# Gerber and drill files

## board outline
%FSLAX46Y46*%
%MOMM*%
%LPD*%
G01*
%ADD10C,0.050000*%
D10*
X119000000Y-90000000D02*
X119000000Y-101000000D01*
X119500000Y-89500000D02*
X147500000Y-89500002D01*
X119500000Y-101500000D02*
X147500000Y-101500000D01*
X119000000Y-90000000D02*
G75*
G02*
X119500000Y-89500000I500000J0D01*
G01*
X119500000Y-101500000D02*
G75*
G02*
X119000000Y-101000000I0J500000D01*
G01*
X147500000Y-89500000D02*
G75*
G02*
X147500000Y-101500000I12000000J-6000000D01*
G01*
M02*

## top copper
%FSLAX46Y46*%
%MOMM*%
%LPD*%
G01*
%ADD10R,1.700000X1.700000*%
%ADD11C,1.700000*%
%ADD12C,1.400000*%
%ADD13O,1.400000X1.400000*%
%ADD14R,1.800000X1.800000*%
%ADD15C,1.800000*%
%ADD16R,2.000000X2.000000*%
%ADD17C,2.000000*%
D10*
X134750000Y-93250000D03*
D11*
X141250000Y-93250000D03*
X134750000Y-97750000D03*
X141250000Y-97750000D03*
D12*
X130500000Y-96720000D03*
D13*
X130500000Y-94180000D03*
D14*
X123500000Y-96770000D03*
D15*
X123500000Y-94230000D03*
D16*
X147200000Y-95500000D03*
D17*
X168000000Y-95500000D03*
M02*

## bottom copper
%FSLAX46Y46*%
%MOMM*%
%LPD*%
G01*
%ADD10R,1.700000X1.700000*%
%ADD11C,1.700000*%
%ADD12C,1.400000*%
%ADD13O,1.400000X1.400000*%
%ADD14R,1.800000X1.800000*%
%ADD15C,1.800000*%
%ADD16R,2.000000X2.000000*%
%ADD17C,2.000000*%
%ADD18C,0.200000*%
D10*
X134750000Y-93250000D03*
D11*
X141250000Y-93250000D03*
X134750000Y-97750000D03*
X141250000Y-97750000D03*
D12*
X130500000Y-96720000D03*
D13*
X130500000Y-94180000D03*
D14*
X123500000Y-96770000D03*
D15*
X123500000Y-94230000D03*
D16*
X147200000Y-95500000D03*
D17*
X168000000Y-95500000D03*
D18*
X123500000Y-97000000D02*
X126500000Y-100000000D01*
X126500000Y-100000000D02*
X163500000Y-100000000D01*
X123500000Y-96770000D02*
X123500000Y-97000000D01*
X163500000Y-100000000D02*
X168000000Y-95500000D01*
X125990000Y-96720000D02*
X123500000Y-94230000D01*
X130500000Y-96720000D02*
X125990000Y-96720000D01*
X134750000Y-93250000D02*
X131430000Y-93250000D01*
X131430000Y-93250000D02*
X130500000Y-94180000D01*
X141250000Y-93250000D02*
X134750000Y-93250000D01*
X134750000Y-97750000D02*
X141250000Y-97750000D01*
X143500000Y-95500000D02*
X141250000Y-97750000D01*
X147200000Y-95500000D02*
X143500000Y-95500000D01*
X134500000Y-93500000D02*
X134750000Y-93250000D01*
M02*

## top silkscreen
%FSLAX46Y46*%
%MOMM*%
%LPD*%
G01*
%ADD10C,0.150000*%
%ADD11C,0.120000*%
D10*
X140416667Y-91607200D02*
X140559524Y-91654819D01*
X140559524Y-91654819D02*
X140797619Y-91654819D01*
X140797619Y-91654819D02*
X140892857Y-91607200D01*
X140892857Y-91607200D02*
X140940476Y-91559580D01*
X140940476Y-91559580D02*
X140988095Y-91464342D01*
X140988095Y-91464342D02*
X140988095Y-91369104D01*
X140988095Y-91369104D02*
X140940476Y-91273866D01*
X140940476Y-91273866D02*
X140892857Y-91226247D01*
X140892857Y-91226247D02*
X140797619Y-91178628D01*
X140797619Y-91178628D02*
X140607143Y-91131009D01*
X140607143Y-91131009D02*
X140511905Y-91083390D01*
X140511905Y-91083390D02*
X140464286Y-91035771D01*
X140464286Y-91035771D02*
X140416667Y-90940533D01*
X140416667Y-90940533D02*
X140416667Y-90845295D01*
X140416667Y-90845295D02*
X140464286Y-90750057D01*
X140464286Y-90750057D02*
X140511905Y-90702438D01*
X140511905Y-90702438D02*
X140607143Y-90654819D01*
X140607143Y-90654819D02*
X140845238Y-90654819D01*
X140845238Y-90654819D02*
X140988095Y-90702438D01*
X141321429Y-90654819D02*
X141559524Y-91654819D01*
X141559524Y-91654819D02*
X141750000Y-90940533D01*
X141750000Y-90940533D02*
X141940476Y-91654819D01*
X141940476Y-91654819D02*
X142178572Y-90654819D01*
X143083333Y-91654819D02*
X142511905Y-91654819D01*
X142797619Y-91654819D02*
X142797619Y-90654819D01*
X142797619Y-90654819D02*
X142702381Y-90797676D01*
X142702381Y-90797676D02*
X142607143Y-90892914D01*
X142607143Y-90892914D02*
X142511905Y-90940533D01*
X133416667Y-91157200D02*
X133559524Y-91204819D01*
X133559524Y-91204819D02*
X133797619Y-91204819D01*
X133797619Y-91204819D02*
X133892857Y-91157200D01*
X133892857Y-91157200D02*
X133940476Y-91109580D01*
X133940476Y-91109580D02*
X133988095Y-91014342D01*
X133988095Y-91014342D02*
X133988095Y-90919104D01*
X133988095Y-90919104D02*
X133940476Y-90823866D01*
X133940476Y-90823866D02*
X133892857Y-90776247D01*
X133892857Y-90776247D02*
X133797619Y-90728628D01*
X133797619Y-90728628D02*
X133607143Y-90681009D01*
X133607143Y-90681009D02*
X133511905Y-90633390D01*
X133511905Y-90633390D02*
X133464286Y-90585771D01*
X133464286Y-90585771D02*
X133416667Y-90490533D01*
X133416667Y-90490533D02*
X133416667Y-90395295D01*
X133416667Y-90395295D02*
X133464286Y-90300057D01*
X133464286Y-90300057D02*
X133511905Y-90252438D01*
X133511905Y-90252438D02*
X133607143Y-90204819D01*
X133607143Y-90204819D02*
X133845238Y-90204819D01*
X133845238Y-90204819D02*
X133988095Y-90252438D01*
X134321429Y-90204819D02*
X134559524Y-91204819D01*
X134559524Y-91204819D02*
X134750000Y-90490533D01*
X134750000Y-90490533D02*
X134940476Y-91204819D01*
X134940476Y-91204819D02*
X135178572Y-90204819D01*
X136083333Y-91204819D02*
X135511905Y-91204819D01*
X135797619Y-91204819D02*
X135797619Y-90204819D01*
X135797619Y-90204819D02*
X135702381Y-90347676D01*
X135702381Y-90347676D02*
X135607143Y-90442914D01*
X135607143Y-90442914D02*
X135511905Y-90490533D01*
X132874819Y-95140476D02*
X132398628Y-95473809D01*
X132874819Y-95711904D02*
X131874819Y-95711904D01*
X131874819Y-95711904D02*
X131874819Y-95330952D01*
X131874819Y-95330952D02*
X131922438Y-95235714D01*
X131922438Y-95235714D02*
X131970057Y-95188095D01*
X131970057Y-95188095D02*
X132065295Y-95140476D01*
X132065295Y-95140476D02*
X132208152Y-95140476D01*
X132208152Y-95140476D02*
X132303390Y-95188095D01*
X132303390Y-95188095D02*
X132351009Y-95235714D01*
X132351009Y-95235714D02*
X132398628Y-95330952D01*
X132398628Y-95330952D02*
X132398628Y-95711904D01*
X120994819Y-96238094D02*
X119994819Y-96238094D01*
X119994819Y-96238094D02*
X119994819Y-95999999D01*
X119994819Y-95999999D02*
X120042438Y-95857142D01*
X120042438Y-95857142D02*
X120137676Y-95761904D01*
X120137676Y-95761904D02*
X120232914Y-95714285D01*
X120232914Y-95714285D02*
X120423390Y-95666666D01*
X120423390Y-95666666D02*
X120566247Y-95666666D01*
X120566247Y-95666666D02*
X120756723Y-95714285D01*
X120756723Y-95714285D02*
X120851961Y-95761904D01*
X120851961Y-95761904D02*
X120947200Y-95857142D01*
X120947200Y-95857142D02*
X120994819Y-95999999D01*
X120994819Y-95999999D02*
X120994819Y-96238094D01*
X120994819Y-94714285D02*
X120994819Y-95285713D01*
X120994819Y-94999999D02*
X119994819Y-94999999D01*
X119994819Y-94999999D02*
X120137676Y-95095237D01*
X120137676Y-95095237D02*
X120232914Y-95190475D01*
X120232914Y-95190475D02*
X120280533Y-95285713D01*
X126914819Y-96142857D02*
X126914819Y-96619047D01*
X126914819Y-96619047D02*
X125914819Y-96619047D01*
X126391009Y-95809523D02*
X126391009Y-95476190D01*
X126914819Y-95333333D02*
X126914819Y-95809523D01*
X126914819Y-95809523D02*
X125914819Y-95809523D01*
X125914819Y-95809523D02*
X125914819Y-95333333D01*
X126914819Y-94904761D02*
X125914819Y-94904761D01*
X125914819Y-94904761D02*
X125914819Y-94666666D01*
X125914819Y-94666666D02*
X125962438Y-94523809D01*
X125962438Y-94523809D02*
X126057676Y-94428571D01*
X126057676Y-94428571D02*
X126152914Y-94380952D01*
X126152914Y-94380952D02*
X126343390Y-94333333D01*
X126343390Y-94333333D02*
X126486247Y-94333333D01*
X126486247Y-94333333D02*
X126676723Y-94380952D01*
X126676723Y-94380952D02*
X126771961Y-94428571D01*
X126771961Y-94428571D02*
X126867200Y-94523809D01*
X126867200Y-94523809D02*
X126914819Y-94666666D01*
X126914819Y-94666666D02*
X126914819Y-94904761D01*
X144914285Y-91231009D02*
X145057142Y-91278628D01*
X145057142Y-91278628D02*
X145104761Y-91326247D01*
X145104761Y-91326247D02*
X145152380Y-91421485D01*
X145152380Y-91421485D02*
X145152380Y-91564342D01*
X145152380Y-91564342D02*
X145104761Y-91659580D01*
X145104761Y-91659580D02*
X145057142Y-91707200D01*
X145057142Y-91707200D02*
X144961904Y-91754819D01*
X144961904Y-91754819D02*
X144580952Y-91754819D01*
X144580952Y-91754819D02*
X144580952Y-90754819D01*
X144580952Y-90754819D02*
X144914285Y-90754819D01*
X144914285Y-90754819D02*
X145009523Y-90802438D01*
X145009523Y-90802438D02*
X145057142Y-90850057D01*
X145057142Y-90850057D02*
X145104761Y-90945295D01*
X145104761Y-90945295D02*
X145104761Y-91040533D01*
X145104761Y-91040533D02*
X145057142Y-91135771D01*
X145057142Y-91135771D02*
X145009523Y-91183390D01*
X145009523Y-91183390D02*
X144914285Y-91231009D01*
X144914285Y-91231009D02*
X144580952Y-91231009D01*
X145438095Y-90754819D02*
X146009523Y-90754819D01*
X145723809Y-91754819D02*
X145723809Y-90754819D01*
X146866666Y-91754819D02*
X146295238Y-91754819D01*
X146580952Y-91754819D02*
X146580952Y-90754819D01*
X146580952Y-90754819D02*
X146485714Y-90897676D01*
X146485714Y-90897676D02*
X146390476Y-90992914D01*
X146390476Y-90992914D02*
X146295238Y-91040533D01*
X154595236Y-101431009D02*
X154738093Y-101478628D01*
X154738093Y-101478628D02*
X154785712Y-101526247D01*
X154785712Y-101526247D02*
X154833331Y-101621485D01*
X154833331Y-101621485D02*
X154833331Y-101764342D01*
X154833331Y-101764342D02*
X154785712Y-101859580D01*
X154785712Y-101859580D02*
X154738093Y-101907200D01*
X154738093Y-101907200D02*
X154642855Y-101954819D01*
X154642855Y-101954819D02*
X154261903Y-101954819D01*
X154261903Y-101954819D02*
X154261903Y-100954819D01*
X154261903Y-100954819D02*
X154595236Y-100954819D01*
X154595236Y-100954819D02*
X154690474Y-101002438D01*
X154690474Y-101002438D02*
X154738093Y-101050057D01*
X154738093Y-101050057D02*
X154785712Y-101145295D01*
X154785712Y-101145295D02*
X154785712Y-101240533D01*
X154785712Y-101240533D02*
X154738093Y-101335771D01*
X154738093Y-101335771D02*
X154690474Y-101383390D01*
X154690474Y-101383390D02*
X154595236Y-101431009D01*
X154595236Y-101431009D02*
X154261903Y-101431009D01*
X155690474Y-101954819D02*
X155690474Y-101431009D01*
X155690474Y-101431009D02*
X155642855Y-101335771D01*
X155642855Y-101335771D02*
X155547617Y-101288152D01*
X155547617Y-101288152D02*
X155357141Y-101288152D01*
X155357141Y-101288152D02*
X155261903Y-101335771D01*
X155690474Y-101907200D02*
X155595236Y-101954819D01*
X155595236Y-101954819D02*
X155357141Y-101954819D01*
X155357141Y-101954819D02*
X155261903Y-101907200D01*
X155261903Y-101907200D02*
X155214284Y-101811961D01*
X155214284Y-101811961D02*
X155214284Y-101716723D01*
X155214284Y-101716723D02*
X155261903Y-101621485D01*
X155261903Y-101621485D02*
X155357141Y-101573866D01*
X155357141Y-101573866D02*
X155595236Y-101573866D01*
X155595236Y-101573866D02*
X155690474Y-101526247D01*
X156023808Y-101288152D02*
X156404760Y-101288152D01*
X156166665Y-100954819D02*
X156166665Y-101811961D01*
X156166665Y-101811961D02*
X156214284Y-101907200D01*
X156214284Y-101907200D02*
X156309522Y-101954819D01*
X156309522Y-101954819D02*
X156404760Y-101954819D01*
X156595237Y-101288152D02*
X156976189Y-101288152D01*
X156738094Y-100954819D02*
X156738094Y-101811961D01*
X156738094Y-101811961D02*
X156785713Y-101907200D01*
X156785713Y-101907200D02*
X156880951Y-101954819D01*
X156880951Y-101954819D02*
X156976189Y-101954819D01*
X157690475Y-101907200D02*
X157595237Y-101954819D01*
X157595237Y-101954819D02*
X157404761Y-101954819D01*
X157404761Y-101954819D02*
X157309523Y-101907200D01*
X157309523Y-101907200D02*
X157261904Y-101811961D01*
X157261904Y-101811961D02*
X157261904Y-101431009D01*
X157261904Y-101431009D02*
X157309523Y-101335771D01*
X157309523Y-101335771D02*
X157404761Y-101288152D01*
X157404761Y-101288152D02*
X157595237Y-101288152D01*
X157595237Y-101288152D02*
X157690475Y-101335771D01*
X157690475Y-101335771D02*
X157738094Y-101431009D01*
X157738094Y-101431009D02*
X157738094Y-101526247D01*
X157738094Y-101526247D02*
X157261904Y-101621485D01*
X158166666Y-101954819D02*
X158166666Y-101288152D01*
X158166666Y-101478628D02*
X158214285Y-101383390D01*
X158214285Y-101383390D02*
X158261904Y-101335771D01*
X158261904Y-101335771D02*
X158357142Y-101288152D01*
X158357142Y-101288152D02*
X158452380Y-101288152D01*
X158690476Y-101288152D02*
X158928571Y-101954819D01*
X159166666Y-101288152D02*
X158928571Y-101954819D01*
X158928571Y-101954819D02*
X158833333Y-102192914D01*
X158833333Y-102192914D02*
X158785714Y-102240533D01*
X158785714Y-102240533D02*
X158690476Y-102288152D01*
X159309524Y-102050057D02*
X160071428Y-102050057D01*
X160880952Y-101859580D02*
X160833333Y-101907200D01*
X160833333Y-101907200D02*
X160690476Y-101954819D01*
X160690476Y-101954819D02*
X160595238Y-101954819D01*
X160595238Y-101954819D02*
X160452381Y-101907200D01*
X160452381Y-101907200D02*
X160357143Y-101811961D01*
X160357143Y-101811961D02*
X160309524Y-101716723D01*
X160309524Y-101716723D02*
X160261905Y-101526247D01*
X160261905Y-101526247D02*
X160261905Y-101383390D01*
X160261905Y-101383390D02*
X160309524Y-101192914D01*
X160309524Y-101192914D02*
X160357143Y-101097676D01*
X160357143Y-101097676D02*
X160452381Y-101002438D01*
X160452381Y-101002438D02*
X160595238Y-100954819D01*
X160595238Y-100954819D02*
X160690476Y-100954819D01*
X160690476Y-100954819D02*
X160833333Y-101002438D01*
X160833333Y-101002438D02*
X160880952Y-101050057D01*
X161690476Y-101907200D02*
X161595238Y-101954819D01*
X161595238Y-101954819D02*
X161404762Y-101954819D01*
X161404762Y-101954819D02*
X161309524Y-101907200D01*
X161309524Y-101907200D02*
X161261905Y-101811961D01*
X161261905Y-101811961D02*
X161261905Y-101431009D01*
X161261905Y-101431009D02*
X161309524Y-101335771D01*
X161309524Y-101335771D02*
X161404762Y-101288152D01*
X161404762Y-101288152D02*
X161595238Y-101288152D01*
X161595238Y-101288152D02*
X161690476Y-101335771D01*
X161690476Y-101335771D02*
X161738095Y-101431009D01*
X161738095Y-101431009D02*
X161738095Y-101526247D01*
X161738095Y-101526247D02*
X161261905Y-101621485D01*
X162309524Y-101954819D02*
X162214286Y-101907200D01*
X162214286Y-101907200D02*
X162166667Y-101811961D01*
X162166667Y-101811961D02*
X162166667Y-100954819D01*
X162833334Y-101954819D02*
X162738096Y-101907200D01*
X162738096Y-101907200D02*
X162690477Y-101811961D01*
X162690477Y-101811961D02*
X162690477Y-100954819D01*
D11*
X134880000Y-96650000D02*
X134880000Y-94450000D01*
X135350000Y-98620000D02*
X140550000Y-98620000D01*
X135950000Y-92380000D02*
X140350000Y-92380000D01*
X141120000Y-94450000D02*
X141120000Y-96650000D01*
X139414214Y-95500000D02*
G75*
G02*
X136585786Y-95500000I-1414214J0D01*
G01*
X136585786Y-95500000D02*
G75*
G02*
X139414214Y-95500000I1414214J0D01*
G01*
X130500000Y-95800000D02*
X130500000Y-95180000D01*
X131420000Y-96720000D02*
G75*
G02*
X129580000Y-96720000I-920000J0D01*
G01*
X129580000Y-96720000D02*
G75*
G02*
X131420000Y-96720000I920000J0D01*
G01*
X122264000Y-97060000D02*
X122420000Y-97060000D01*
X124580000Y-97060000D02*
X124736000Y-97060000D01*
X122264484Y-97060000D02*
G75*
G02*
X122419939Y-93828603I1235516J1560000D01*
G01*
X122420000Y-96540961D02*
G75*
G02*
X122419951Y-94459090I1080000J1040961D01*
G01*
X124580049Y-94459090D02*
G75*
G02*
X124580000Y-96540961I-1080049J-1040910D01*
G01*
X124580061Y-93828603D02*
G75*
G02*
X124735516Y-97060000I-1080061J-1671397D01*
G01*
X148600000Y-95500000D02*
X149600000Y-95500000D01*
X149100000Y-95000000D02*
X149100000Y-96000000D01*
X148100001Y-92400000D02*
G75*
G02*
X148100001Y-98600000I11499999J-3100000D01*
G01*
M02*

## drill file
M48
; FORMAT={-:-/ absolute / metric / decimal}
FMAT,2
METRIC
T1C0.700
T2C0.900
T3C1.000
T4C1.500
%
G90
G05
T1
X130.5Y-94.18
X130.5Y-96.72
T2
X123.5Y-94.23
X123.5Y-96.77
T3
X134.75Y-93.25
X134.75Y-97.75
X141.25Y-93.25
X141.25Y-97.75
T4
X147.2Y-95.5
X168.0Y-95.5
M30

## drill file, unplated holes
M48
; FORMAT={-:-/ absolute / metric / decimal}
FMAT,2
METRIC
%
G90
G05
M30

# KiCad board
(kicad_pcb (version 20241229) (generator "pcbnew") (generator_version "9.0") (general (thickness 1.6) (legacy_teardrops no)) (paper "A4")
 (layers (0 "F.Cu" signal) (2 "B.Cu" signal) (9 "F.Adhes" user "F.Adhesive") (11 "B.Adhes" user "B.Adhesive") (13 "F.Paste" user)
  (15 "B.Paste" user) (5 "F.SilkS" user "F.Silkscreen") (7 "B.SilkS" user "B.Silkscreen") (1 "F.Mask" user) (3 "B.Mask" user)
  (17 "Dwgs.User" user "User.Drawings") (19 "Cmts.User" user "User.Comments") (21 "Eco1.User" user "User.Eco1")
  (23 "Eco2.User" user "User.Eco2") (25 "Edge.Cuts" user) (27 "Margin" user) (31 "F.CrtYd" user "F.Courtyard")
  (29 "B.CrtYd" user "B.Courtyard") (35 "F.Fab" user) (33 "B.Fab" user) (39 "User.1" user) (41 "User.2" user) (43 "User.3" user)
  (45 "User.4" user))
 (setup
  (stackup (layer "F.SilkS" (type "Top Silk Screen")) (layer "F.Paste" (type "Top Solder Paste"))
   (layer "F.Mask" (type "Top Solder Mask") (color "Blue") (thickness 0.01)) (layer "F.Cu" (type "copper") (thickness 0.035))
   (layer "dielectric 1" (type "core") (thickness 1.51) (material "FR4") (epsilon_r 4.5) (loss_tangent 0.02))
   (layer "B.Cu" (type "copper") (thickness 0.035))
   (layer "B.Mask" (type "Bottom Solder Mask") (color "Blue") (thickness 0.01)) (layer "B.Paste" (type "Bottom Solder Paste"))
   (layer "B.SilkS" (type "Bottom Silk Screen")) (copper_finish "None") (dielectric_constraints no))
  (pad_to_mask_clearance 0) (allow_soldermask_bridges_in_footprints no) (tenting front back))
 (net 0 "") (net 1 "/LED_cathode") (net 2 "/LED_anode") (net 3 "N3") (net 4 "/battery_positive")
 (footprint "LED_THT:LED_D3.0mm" (layer "F.Cu") (at 123.5 96.77 90)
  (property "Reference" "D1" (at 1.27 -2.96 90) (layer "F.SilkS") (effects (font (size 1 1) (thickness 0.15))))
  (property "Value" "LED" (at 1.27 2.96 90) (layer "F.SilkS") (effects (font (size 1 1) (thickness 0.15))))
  (fp_line (start -0.29 -1.236) (end -0.29 -1.08) (stroke (width 0.12) (type solid)) (layer "F.SilkS"))
  (fp_line (start -0.29 1.08) (end -0.29 1.236) (stroke (width 0.12) (type solid)) (layer "F.SilkS"))
  (fp_arc (start -0.29 -1.235516) (mid 1.365624 -1.987701) (end 2.941397 -1.080061) (stroke (width 0.12) (type solid)) (layer "F.SilkS"))
  (fp_arc (start 0.229039 -1.08) (mid 1.269964 -1.5) (end 2.31091 -1.080049) (stroke (width 0.12) (type solid)) (layer "F.SilkS"))
  (fp_arc (start 2.31091 1.080049) (mid 1.269964 1.5) (end 0.229039 1.08) (stroke (width 0.12) (type solid)) (layer "F.SilkS"))
  (fp_arc (start 2.941397 1.080061) (mid 1.365624 1.987701) (end -0.29 1.235516) (stroke (width 0.12) (type solid)) (layer "F.SilkS"))
  (pad "1" thru_hole rect (at 0 0 90) (size 1.8 1.8) (drill 0.9) (layers "*.Cu" "*.Mask") (remove_unused_layers no) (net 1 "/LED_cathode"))
  (pad "2" thru_hole circle (at 2.54 0 90) (size 1.8 1.8) (drill 0.9) (layers "*.Cu" "*.Mask") (remove_unused_layers no)
   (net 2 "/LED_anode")))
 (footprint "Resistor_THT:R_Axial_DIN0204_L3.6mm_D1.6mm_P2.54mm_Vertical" (layer "F.Cu") (at 130.5 96.72 90)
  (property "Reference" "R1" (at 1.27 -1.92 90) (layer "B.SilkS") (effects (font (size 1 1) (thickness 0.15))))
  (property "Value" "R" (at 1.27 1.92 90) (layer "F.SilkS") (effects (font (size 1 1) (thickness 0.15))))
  (fp_line (start 0.92 0) (end 1.54 0) (stroke (width 0.12) (type solid)) (layer "F.SilkS"))
  (fp_circle (center 0 0) (end 0.92 0) (stroke (width 0.12) (type solid)) (fill no) (layer "F.SilkS"))
  (pad "1" thru_hole circle (at 0 0 90) (size 1.4 1.4) (drill 0.7) (layers "*.Cu" "*.Mask") (remove_unused_layers no) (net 2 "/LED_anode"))
  (pad "2" thru_hole oval (at 2.54 0 90) (size 1.4 1.4) (drill 0.7) (layers "*.Cu" "*.Mask") (remove_unused_layers no) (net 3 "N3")))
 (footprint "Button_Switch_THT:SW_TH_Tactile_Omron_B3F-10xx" (layer "F.Cu") (at 134.75 93.25)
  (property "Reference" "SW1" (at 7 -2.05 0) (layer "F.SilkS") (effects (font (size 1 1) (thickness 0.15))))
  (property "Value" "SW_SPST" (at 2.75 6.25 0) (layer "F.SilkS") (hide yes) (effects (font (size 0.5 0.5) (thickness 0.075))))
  (fp_line (start 0.13 3.4) (end 0.13 1.2) (stroke (width 0.12) (type solid)) (layer "F.SilkS"))
  (fp_line (start 0.6 5.37) (end 5.8 5.37) (stroke (width 0.12) (type solid)) (layer "F.SilkS"))
  (fp_line (start 1.2 -0.87) (end 5.6 -0.87) (stroke (width 0.12) (type solid)) (layer "F.SilkS"))
  (fp_line (start 6.37 1.2) (end 6.37 3.4) (stroke (width 0.12) (type solid)) (layer "F.SilkS"))
  (fp_circle (center 3.25 2.25) (end 4.25 3.25) (stroke (width 0.12) (type solid)) (fill no) (layer "F.SilkS"))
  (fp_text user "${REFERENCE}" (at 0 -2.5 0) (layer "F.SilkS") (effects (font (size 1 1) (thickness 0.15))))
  (pad "1" thru_hole rect (at 0 0) (size 1.7 1.7) (drill 1) (layers "*.Cu" "*.Mask") (remove_unused_layers no) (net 3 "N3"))
  (pad "1" thru_hole circle (at 6.5 0) (size 1.7 1.7) (drill 1) (layers "*.Cu" "*.Mask") (remove_unused_layers no) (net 3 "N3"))
  (pad "2" thru_hole circle (at 0 4.5) (size 1.7 1.7) (drill 1) (layers "*.Cu" "*.Mask") (remove_unused_layers no)
   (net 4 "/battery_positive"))
  (pad "2" thru_hole circle (at 6.5 4.5) (size 1.7 1.7) (drill 1) (layers "*.Cu" "*.Mask") (remove_unused_layers no)
   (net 4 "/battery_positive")))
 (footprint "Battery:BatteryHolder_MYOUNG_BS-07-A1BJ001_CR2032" (layer "F.Cu") (at 147.2 95.5)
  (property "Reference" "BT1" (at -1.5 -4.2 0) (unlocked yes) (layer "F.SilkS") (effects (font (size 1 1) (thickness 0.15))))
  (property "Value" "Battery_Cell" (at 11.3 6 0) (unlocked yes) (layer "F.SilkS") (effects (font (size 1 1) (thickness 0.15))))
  (fp_line (start 1.4 0) (end 2.4 0) (stroke (width 0.12) (type default)) (layer "F.SilkS"))
  (fp_line (start 1.9 -0.5) (end 1.9 0.5) (stroke (width 0.12) (type default)) (layer "F.SilkS"))
  (fp_arc (start 0.900001 -3.1) (mid 24.310499 0) (end 0.900001 3.1) (stroke (width 0.12) (type default)) (layer "F.SilkS"))
  (pad "1" thru_hole rect (at 0 0 180) (size 2 2) (drill 1.5) (layers "*.Cu" "*.Mask") (remove_unused_layers no) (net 4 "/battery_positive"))
  (pad "2" thru_hole circle (at 20.8 0 180) (size 2 2) (drill 1.5) (layers "*.Cu" "*.Mask") (remove_unused_layers no) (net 1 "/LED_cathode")))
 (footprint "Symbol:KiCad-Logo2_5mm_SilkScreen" (layer "B.Cu") (at 159.5 95 180)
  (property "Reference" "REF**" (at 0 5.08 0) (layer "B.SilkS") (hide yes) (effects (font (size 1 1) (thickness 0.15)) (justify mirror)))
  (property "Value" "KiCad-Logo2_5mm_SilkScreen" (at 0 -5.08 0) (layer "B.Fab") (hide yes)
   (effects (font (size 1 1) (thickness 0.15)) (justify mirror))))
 (gr_line (start 119.5 101.5) (end 147.5 101.5) (stroke (width 0.05) (type default)) (layer "Edge.Cuts"))
 (gr_line (start 119 90) (end 119 101) (stroke (width 0.05) (type default)) (layer "Edge.Cuts"))
 (gr_arc (start 119 90) (mid 119.146447 89.646447) (end 119.5 89.5) (stroke (width 0.05) (type default)) (layer "Edge.Cuts"))
 (gr_arc (start 119.5 101.5) (mid 119.146447 101.353553) (end 119 101) (stroke (width 0.05) (type default)) (layer "Edge.Cuts"))
 (gr_arc (start 147.5 89.5) (mid 172.916408 95.5) (end 147.5 101.5) (stroke (width 0.05) (type default)) (layer "Edge.Cuts"))
 (gr_line (start 119.5 89.5) (end 147.5 89.500002) (stroke (width 0.05) (type default)) (layer "Edge.Cuts"))
 (segment (start 134.75 97.75) (end 141.25 97.75) (width 0.2) (layer "B.Cu") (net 4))
 (segment (start 143.5 95.5) (end 141.25 97.75) (width 0.2) (layer "B.Cu") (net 4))
 (segment (start 147.2 95.5) (end 143.5 95.5) (width 0.2) (layer "B.Cu") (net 4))
 (segment (start 123.5 97) (end 126.5 100) (width 0.2) (layer "B.Cu") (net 1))
 (segment (start 126.5 100) (end 163.5 100) (width 0.2) (layer "B.Cu") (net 1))
 (segment (start 123.5 96.77) (end 123.5 97) (width 0.2) (layer "B.Cu") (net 1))
 (segment (start 163.5 100) (end 168 95.5) (width 0.2) (layer "B.Cu") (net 1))
 (segment (start 125.99 96.72) (end 123.5 94.23) (width 0.2) (layer "B.Cu") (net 2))
 (segment (start 130.5 96.72) (end 125.99 96.72) (width 0.2) (layer "B.Cu") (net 2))
 (segment (start 134.75 93.25) (end 131.43 93.25) (width 0.2) (layer "B.Cu") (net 3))
 (segment (start 131.43 93.25) (end 130.5 94.18) (width 0.2) (layer "B.Cu") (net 3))
 (segment (start 134.5 93.5) (end 134.75 93.25) (width 0.2) (layer "B.Cu") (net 3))
 (segment (start 141.25 93.25) (end 134.75 93.25) (width 0.2) (layer "B.Cu") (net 3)))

